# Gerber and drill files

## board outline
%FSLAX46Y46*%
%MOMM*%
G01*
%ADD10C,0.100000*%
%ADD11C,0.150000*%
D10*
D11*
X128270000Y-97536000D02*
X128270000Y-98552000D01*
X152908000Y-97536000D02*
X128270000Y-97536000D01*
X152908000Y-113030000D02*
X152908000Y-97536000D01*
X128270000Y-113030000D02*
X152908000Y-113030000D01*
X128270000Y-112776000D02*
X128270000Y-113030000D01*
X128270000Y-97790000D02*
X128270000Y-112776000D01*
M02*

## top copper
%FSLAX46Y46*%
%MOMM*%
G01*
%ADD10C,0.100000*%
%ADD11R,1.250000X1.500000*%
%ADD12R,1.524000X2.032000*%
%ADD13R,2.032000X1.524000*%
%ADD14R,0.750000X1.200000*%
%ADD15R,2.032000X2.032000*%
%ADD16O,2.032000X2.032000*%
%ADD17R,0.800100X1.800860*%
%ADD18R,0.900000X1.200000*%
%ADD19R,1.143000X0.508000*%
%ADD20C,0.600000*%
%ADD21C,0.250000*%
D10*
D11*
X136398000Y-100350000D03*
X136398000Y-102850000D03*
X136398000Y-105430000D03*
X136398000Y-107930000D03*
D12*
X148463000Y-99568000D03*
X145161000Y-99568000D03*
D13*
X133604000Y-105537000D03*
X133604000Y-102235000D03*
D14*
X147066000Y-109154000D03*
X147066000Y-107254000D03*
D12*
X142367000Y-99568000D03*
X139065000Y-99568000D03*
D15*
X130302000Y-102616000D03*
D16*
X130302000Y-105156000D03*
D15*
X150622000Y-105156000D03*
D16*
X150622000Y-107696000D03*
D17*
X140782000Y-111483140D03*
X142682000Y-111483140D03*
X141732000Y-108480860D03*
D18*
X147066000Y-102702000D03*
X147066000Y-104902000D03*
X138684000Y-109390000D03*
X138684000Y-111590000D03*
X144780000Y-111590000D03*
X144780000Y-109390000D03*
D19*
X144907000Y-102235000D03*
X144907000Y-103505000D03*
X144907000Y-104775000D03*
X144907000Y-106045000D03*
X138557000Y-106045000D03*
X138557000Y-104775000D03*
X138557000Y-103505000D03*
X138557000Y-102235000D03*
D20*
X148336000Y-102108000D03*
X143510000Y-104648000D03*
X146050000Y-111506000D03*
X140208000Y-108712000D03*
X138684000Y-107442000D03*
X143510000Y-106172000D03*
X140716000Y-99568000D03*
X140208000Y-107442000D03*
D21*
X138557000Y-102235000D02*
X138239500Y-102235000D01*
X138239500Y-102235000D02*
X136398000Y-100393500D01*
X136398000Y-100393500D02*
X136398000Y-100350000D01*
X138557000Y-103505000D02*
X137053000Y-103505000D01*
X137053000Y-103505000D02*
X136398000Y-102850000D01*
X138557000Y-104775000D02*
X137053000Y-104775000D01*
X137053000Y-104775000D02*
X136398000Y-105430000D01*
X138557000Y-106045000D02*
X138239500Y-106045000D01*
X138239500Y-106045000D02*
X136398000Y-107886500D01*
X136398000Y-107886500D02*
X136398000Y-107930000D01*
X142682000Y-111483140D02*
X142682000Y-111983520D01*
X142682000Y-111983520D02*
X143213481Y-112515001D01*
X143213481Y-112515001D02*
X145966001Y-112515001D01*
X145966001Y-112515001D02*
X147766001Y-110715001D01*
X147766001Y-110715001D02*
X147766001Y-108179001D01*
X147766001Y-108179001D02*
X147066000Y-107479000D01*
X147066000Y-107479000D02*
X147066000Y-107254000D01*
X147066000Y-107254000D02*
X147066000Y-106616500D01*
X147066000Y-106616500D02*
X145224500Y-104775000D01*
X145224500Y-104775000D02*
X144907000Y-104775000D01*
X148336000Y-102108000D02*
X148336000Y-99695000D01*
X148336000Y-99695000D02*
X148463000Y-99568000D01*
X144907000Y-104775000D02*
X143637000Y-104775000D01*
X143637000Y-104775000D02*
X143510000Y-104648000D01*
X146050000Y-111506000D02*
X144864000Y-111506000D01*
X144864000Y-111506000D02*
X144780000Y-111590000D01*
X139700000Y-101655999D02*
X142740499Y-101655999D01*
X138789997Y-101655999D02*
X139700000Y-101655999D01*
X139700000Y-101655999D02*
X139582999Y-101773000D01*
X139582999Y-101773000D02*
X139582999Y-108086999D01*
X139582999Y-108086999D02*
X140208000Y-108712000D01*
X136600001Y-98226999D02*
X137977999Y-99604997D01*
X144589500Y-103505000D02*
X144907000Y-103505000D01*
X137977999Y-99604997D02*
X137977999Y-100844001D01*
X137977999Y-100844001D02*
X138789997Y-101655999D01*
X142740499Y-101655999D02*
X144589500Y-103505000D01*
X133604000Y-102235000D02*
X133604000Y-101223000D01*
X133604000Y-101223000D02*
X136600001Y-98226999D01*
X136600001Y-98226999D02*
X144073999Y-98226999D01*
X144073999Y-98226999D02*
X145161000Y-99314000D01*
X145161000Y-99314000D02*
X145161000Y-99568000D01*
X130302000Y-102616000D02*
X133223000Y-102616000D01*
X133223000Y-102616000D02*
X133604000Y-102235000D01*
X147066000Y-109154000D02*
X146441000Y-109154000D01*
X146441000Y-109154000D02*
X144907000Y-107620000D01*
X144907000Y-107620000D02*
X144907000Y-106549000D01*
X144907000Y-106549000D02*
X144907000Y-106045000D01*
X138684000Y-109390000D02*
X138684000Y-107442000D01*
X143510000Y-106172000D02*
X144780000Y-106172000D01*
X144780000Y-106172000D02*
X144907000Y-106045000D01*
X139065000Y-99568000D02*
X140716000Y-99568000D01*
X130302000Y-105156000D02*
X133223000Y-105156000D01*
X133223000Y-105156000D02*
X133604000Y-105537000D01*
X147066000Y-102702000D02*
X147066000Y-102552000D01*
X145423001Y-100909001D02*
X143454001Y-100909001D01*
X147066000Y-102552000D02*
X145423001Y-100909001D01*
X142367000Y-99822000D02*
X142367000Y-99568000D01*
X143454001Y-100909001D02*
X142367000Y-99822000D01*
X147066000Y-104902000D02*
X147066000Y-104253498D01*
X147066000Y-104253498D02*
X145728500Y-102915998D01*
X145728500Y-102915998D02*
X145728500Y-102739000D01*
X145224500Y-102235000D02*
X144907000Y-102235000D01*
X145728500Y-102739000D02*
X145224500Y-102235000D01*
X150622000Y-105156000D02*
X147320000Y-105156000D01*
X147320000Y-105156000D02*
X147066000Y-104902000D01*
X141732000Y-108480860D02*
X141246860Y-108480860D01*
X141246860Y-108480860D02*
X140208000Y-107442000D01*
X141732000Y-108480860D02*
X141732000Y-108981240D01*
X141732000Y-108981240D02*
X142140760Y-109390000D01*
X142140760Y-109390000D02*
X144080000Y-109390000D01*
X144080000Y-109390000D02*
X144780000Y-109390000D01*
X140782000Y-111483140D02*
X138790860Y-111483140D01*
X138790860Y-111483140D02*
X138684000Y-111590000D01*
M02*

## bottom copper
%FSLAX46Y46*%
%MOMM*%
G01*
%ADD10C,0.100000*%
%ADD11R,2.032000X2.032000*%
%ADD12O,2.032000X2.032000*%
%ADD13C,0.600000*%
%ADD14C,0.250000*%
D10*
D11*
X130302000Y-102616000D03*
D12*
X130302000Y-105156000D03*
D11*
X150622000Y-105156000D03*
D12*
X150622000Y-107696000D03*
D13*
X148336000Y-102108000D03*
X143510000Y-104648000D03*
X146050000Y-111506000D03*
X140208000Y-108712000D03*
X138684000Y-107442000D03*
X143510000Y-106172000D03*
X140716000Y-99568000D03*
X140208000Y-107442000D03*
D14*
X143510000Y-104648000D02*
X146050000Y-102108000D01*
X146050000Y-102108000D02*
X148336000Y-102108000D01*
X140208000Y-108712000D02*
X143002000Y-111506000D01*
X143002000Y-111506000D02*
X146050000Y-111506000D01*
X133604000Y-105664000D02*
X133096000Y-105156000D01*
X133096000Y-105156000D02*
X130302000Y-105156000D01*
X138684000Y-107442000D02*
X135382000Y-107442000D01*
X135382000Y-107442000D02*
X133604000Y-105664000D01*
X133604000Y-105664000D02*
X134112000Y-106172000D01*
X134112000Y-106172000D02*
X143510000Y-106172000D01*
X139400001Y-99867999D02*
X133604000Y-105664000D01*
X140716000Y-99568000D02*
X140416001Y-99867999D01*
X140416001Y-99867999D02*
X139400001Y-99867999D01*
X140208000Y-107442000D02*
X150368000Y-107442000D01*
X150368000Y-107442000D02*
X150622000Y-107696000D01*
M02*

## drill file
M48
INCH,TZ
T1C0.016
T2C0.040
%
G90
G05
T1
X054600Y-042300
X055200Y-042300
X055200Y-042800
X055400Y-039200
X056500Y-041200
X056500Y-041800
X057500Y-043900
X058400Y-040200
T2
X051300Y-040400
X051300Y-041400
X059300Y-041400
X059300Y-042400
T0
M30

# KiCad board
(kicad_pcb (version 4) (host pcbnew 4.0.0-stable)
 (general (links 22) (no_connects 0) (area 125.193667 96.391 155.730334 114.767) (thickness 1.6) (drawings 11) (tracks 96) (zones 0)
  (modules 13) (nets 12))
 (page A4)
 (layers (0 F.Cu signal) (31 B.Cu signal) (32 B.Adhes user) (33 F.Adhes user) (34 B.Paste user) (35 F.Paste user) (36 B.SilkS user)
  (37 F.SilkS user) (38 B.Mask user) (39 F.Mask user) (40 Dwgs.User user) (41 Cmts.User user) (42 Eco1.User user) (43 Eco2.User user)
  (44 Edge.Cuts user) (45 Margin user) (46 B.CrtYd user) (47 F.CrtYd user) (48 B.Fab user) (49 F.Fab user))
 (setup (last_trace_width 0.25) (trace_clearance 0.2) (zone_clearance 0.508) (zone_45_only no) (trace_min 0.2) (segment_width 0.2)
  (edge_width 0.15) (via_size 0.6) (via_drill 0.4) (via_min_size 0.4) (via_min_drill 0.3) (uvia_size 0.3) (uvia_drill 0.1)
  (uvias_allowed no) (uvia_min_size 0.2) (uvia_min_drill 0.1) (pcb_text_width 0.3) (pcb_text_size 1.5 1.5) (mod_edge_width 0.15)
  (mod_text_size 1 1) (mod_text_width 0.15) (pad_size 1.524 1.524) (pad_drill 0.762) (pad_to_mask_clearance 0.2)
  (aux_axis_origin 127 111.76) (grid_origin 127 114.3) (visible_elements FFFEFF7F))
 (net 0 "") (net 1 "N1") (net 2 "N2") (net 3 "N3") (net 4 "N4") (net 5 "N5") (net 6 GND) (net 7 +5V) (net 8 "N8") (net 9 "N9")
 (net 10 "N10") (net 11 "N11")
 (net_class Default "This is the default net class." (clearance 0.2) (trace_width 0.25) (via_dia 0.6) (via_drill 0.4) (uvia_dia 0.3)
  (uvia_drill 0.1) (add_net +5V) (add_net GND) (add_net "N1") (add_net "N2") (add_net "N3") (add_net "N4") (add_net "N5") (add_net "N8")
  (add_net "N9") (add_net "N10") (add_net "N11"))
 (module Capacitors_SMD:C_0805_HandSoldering (layer F.Cu) (at 136.398 101.6 270)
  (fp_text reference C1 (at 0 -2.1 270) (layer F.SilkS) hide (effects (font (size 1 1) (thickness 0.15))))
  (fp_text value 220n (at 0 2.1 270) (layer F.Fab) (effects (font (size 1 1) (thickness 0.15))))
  (pad 1 smd rect (at -1.25 0 270) (size 1.5 1.25) (layers F.Cu F.Paste F.Mask) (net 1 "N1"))
  (pad 2 smd rect (at 1.25 0 270) (size 1.5 1.25) (layers F.Cu F.Paste F.Mask) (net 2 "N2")))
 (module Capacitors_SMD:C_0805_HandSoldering (layer F.Cu) (at 136.398 106.68 270)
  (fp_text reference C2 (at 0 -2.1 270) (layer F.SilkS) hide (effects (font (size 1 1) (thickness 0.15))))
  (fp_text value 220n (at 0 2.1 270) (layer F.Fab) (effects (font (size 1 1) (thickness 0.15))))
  (pad 1 smd rect (at -1.25 0 270) (size 1.5 1.25) (layers F.Cu F.Paste F.Mask) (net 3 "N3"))
  (pad 2 smd rect (at 1.25 0 270) (size 1.5 1.25) (layers F.Cu F.Paste F.Mask) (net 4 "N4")))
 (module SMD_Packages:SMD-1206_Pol (layer F.Cu) (at 146.812 99.568 180)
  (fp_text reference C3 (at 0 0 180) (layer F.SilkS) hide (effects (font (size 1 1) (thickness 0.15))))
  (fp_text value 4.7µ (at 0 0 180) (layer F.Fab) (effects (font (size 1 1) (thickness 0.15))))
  (pad 1 smd rect (at -1.651 0 180) (size 1.524 2.032) (layers F.Cu F.Paste F.Mask) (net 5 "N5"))
  (pad 2 smd rect (at 1.651 0 180) (size 1.524 2.032) (layers F.Cu F.Paste F.Mask) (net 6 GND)))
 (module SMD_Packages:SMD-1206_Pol (layer F.Cu) (at 133.604 103.886 90)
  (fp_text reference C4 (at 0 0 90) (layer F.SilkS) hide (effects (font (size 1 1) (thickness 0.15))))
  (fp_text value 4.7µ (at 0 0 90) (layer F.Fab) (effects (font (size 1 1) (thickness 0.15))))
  (pad 1 smd rect (at -1.651 0 90) (size 1.524 2.032) (layers F.Cu F.Paste F.Mask) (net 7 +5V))
  (pad 2 smd rect (at 1.651 0 90) (size 1.524 2.032) (layers F.Cu F.Paste F.Mask) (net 6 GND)))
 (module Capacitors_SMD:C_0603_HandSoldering (layer F.Cu) (at 147.066 108.204 90)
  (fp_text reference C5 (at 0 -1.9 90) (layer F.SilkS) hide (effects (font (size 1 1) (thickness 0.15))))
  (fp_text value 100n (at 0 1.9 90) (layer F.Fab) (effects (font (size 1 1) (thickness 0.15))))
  (pad 1 smd rect (at -0.95 0 90) (size 1.2 0.75) (layers F.Cu F.Paste F.Mask) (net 7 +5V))
  (pad 2 smd rect (at 0.95 0 90) (size 1.2 0.75) (layers F.Cu F.Paste F.Mask) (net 5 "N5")))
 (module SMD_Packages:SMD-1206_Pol (layer F.Cu) (at 140.716 99.568 180)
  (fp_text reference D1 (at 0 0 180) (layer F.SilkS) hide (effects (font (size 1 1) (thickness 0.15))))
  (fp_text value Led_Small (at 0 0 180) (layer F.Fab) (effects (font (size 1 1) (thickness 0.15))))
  (pad 1 smd rect (at -1.651 0 180) (size 1.524 2.032) (layers F.Cu F.Paste F.Mask) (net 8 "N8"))
  (pad 2 smd rect (at 1.651 0 180) (size 1.524 2.032) (layers F.Cu F.Paste F.Mask) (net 7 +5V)))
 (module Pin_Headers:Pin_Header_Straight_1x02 (layer F.Cu) (at 130.302 102.616)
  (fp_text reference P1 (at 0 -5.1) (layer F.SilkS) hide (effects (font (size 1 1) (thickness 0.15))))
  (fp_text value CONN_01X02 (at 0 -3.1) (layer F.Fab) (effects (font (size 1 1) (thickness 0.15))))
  (pad 1 thru_hole rect (at 0 0) (size 2.032 2.032) (drill 1.016) (layers *.Cu *.Mask F.SilkS) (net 6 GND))
  (pad 2 thru_hole oval (at 0 2.54) (size 2.032 2.032) (drill 1.016) (layers *.Cu *.Mask F.SilkS) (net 7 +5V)))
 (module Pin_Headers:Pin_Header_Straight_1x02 (layer F.Cu) (at 150.622 105.156)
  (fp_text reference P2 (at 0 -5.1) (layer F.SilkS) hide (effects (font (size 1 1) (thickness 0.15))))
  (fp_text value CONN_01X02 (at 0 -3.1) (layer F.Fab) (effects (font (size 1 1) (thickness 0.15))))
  (pad 1 thru_hole rect (at 0 0) (size 2.032 2.032) (drill 1.016) (layers *.Cu *.Mask F.SilkS) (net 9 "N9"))
  (pad 2 thru_hole oval (at 0 2.54) (size 2.032 2.032) (drill 1.016) (layers *.Cu *.Mask F.SilkS) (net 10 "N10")))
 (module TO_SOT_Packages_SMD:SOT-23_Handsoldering (layer F.Cu) (at 141.732 109.982)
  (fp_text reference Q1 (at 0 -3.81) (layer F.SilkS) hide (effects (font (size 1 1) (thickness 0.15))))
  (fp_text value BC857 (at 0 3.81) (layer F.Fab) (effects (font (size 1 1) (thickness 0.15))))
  (pad 1 smd rect (at -0.95 1.50114) (size 0.8001 1.80086) (layers F.Cu F.Paste F.Mask) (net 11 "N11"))
  (pad 2 smd rect (at 0.95 1.50114) (size 0.8001 1.80086) (layers F.Cu F.Paste F.Mask) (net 5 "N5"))
  (pad 3 smd rect (at 0 -1.50114) (size 0.8001 1.80086) (layers F.Cu F.Paste F.Mask) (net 10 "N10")))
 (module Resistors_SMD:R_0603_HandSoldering (layer F.Cu) (at 147.066 103.802 270)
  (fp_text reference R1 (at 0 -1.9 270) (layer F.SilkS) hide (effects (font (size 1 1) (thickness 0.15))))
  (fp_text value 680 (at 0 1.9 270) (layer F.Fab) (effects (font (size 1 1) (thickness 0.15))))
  (pad 1 smd rect (at -1.1 0 270) (size 1.2 0.9) (layers F.Cu F.Paste F.Mask) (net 8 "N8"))
  (pad 2 smd rect (at 1.1 0 270) (size 1.2 0.9) (layers F.Cu F.Paste F.Mask) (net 9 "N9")))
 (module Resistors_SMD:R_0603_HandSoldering (layer F.Cu) (at 138.684 110.49 270)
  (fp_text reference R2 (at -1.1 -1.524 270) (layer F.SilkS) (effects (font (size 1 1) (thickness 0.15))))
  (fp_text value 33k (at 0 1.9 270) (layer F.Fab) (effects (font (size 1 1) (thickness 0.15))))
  (pad 1 smd rect (at -1.1 0 270) (size 1.2 0.9) (layers F.Cu F.Paste F.Mask) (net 7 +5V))
  (pad 2 smd rect (at 1.1 0 270) (size 1.2 0.9) (layers F.Cu F.Paste F.Mask) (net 11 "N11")))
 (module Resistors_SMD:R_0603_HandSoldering (layer F.Cu) (at 144.78 110.49 90)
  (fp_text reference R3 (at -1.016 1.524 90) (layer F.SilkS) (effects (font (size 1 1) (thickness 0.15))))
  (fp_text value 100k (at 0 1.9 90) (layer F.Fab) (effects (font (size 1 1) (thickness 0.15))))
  (pad 1 smd rect (at -1.1 0 90) (size 1.2 0.9) (layers F.Cu F.Paste F.Mask) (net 6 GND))
  (pad 2 smd rect (at 1.1 0 90) (size 1.2 0.9) (layers F.Cu F.Paste F.Mask) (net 10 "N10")))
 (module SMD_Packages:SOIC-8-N (layer F.Cu) (at 141.732 104.14 270)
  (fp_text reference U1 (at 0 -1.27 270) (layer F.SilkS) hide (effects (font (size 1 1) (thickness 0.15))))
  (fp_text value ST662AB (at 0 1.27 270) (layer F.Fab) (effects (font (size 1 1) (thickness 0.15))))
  (pad 8 smd rect (at -1.905 -3.175 270) (size 0.508 1.143) (layers F.Cu F.Paste F.Mask) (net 9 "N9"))
  (pad 7 smd rect (at -0.635 -3.175 270) (size 0.508 1.143) (layers F.Cu F.Paste F.Mask) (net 6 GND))
  (pad 6 smd rect (at 0.635 -3.175 270) (size 0.508 1.143) (layers F.Cu F.Paste F.Mask) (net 5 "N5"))
  (pad 5 smd rect (at 1.905 -3.175 270) (size 0.508 1.143) (layers F.Cu F.Paste F.Mask) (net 7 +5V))
  (pad 4 smd rect (at 1.905 3.175 270) (size 0.508 1.143) (layers F.Cu F.Paste F.Mask) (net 4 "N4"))
  (pad 3 smd rect (at 0.635 3.175 270) (size 0.508 1.143) (layers F.Cu F.Paste F.Mask) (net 3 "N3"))
  (pad 2 smd rect (at -0.635 3.175 270) (size 0.508 1.143) (layers F.Cu F.Paste F.Mask) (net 2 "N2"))
  (pad 1 smd rect (at -1.905 3.175 270) (size 0.508 1.143) (layers F.Cu F.Paste F.Mask) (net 1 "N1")))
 (gr_line (start 128.27 97.536) (end 128.27 98.552) (layer Edge.Cuts) (width 0.15))
 (gr_line (start 152.908 97.536) (end 128.27 97.536) (layer Edge.Cuts) (width 0.15))
 (gr_line (start 152.908 113.03) (end 152.908 97.536) (layer Edge.Cuts) (width 0.15))
 (gr_line (start 128.27 113.03) (end 152.908 113.03) (layer Edge.Cuts) (width 0.15))
 (gr_line (start 128.27 112.776) (end 128.27 113.03) (layer Edge.Cuts) (width 0.15))
 (gr_line (start 128.27 97.79) (end 128.27 112.776) (layer Edge.Cuts) (width 0.15))
 (segment (start 138.557 102.235) (end 138.2395 102.235) (width 0.25) (layer F.Cu) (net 1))
 (segment (start 138.2395 102.235) (end 136.398 100.3935) (width 0.25) (layer F.Cu) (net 1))
 (segment (start 136.398 100.3935) (end 136.398 100.35) (width 0.25) (layer F.Cu) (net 1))
 (segment (start 138.557 103.505) (end 137.053 103.505) (width 0.25) (layer F.Cu) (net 2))
 (segment (start 137.053 103.505) (end 136.398 102.85) (width 0.25) (layer F.Cu) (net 2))
 (segment (start 138.557 104.775) (end 137.053 104.775) (width 0.25) (layer F.Cu) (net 3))
 (segment (start 137.053 104.775) (end 136.398 105.43) (width 0.25) (layer F.Cu) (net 3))
 (segment (start 138.557 106.045) (end 138.2395 106.045) (width 0.25) (layer F.Cu) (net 4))
 (segment (start 138.2395 106.045) (end 136.398 107.8865) (width 0.25) (layer F.Cu) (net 4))
 (segment (start 136.398 107.8865) (end 136.398 107.93) (width 0.25) (layer F.Cu) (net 4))
 (segment (start 142.682 111.48314) (end 142.682 111.98352) (width 0.25) (layer F.Cu) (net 5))
 (segment (start 142.682 111.98352) (end 143.213481 112.515001) (width 0.25) (layer F.Cu) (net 5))
 (segment (start 143.213481 112.515001) (end 145.966001 112.515001) (width 0.25) (layer F.Cu) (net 5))
 (segment (start 145.966001 112.515001) (end 147.766001 110.715001) (width 0.25) (layer F.Cu) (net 5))
 (segment (start 147.766001 110.715001) (end 147.766001 108.179001) (width 0.25) (layer F.Cu) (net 5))
 (segment (start 147.766001 108.179001) (end 147.066 107.479) (width 0.25) (layer F.Cu) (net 5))
 (segment (start 147.066 107.479) (end 147.066 107.254) (width 0.25) (layer F.Cu) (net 5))
 (segment (start 147.066 107.254) (end 147.066 106.6165) (width 0.25) (layer F.Cu) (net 5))
 (segment (start 147.066 106.6165) (end 145.2245 104.775) (width 0.25) (layer F.Cu) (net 5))
 (segment (start 145.2245 104.775) (end 144.907 104.775) (width 0.25) (layer F.Cu) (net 5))
 (segment (start 148.336 102.108) (end 148.336 99.695) (width 0.25) (layer F.Cu) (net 5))
 (segment (start 148.336 99.695) (end 148.463 99.568) (width 0.25) (layer F.Cu) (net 5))
 (segment (start 143.51 104.648) (end 146.05 102.108) (width 0.25) (layer B.Cu) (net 5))
 (segment (start 146.05 102.108) (end 148.336 102.108) (width 0.25) (layer B.Cu) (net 5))
 (via (at 148.336 102.108) (size 0.6) (drill 0.4) (layers F.Cu B.Cu) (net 5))
 (segment (start 144.907 104.775) (end 143.637 104.775) (width 0.25) (layer F.Cu) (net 5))
 (segment (start 143.637 104.775) (end 143.51 104.648) (width 0.25) (layer F.Cu) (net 5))
 (via (at 143.51 104.648) (size 0.6) (drill 0.4) (layers F.Cu B.Cu) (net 5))
 (segment (start 146.05 111.506) (end 144.864 111.506) (width 0.25) (layer F.Cu) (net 6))
 (segment (start 144.864 111.506) (end 144.78 111.59) (width 0.25) (layer F.Cu) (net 6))
 (segment (start 140.208 108.712) (end 143.002 111.506) (width 0.25) (layer B.Cu) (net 6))
 (segment (start 143.002 111.506) (end 146.05 111.506) (width 0.25) (layer B.Cu) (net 6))
 (via (at 146.05 111.506) (size 0.6) (drill 0.4) (layers F.Cu B.Cu) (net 6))
 (segment (start 139.7 101.655999) (end 142.740499 101.655999) (width 0.25) (layer F.Cu) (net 6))
 (segment (start 138.789997 101.655999) (end 139.7 101.655999) (width 0.25) (layer F.Cu) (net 6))
 (segment (start 139.7 101.655999) (end 139.582999 101.773) (width 0.25) (layer F.Cu) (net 6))
 (segment (start 139.582999 101.773) (end 139.582999 108.086999) (width 0.25) (layer F.Cu) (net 6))
 (segment (start 139.582999 108.086999) (end 140.208 108.712) (width 0.25) (layer F.Cu) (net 6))
 (via (at 140.208 108.712) (size 0.6) (drill 0.4) (layers F.Cu B.Cu) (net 6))
 (segment (start 136.600001 98.226999) (end 137.977999 99.604997) (width 0.25) (layer F.Cu) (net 6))
 (segment (start 144.5895 103.505) (end 144.907 103.505) (width 0.25) (layer F.Cu) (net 6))
 (segment (start 137.977999 99.604997) (end 137.977999 100.844001) (width 0.25) (layer F.Cu) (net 6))
 (segment (start 137.977999 100.844001) (end 138.789997 101.655999) (width 0.25) (layer F.Cu) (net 6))
 (segment (start 142.740499 101.655999) (end 144.5895 103.505) (width 0.25) (layer F.Cu) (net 6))
 (segment (start 133.604 102.235) (end 133.604 101.223) (width 0.25) (layer F.Cu) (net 6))
 (segment (start 133.604 101.223) (end 136.600001 98.226999) (width 0.25) (layer F.Cu) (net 6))
 (segment (start 136.600001 98.226999) (end 144.073999 98.226999) (width 0.25) (layer F.Cu) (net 6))
 (segment (start 144.073999 98.226999) (end 145.161 99.314) (width 0.25) (layer F.Cu) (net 6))
 (segment (start 145.161 99.314) (end 145.161 99.568) (width 0.25) (layer F.Cu) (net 6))
 (segment (start 130.302 102.616) (end 133.223 102.616) (width 0.25) (layer F.Cu) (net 6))
 (segment (start 133.223 102.616) (end 133.604 102.235) (width 0.25) (layer F.Cu) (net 6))
 (segment (start 147.066 109.154) (end 146.441 109.154) (width 0.25) (layer F.Cu) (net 7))
 (segment (start 146.441 109.154) (end 144.907 107.62) (width 0.25) (layer F.Cu) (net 7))
 (segment (start 144.907 107.62) (end 144.907 106.549) (width 0.25) (layer F.Cu) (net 7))
 (segment (start 144.907 106.549) (end 144.907 106.045) (width 0.25) (layer F.Cu) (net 7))
 (segment (start 133.604 105.664) (end 133.096 105.156) (width 0.25) (layer B.Cu) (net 7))
 (segment (start 133.096 105.156) (end 130.302 105.156) (width 0.25) (layer B.Cu) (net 7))
 (segment (start 138.684 107.442) (end 135.382 107.442) (width 0.25) (layer B.Cu) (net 7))
 (segment (start 135.382 107.442) (end 133.604 105.664) (width 0.25) (layer B.Cu) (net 7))
 (segment (start 138.684 109.39) (end 138.684 107.442) (width 0.25) (layer F.Cu) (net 7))
 (via (at 138.684 107.442) (size 0.6) (drill 0.4) (layers F.Cu B.Cu) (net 7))
 (segment (start 143.51 106.172) (end 144.78 106.172) (width 0.25) (layer F.Cu) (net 7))
 (segment (start 144.78 106.172) (end 144.907 106.045) (width 0.25) (layer F.Cu) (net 7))
 (segment (start 133.604 105.664) (end 134.112 106.172) (width 0.25) (layer B.Cu) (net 7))
 (segment (start 134.112 106.172) (end 143.51 106.172) (width 0.25) (layer B.Cu) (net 7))
 (via (at 143.51 106.172) (size 0.6) (drill 0.4) (layers F.Cu B.Cu) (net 7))
 (segment (start 139.400001 99.867999) (end 133.604 105.664) (width 0.25) (layer B.Cu) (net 7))
 (segment (start 140.716 99.568) (end 140.416001 99.867999) (width 0.25) (layer B.Cu) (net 7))
 (segment (start 140.416001 99.867999) (end 139.400001 99.867999) (width 0.25) (layer B.Cu) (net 7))
 (segment (start 139.065 99.568) (end 140.716 99.568) (width 0.25) (layer F.Cu) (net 7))
 (via (at 140.716 99.568) (size 0.6) (drill 0.4) (layers F.Cu B.Cu) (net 7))
 (segment (start 130.302 105.156) (end 133.223 105.156) (width 0.25) (layer F.Cu) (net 7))
 (segment (start 133.223 105.156) (end 133.604 105.537) (width 0.25) (layer F.Cu) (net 7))
 (segment (start 147.066 102.702) (end 147.066 102.552) (width 0.25) (layer F.Cu) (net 8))
 (segment (start 145.423001 100.909001) (end 143.454001 100.909001) (width 0.25) (layer F.Cu) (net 8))
 (segment (start 147.066 102.552) (end 145.423001 100.909001) (width 0.25) (layer F.Cu) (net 8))
 (segment (start 142.367 99.822) (end 142.367 99.568) (width 0.25) (layer F.Cu) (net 8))
 (segment (start 143.454001 100.909001) (end 142.367 99.822) (width 0.25) (layer F.Cu) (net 8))
 (segment (start 147.066 104.902) (end 147.066 104.253498) (width 0.25) (layer F.Cu) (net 9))
 (segment (start 147.066 104.253498) (end 145.7285 102.915998) (width 0.25) (layer F.Cu) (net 9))
 (segment (start 145.7285 102.915998) (end 145.7285 102.739) (width 0.25) (layer F.Cu) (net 9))
 (segment (start 145.2245 102.235) (end 144.907 102.235) (width 0.25) (layer F.Cu) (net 9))
 (segment (start 145.7285 102.739) (end 145.2245 102.235) (width 0.25) (layer F.Cu) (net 9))
 (segment (start 150.622 105.156) (end 147.32 105.156) (width 0.25) (layer F.Cu) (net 9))
 (segment (start 147.32 105.156) (end 147.066 104.902) (width 0.25) (layer F.Cu) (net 9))
 (segment (start 140.208 107.442) (end 150.368 107.442) (width 0.25) (layer B.Cu) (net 10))
 (segment (start 150.368 107.442) (end 150.622 107.696) (width 0.25) (layer B.Cu) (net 10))
 (segment (start 141.732 108.48086) (end 141.24686 108.48086) (width 0.25) (layer F.Cu) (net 10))
 (segment (start 141.24686 108.48086) (end 140.208 107.442) (width 0.25) (layer F.Cu) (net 10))
 (via (at 140.208 107.442) (size 0.6) (drill 0.4) (layers F.Cu B.Cu) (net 10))
 (segment (start 141.732 108.48086) (end 141.732 108.98124) (width 0.25) (layer F.Cu) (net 10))
 (segment (start 141.732 108.98124) (end 142.14076 109.39) (width 0.25) (layer F.Cu) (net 10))
 (segment (start 142.14076 109.39) (end 144.08 109.39) (width 0.25) (layer F.Cu) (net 10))
 (segment (start 144.08 109.39) (end 144.78 109.39) (width 0.25) (layer F.Cu) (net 10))
 (segment (start 140.782 111.48314) (end 138.79086 111.48314) (width 0.25) (layer F.Cu) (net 11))
 (segment (start 138.79086 111.48314) (end 138.684 111.59) (width 0.25) (layer F.Cu) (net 11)))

